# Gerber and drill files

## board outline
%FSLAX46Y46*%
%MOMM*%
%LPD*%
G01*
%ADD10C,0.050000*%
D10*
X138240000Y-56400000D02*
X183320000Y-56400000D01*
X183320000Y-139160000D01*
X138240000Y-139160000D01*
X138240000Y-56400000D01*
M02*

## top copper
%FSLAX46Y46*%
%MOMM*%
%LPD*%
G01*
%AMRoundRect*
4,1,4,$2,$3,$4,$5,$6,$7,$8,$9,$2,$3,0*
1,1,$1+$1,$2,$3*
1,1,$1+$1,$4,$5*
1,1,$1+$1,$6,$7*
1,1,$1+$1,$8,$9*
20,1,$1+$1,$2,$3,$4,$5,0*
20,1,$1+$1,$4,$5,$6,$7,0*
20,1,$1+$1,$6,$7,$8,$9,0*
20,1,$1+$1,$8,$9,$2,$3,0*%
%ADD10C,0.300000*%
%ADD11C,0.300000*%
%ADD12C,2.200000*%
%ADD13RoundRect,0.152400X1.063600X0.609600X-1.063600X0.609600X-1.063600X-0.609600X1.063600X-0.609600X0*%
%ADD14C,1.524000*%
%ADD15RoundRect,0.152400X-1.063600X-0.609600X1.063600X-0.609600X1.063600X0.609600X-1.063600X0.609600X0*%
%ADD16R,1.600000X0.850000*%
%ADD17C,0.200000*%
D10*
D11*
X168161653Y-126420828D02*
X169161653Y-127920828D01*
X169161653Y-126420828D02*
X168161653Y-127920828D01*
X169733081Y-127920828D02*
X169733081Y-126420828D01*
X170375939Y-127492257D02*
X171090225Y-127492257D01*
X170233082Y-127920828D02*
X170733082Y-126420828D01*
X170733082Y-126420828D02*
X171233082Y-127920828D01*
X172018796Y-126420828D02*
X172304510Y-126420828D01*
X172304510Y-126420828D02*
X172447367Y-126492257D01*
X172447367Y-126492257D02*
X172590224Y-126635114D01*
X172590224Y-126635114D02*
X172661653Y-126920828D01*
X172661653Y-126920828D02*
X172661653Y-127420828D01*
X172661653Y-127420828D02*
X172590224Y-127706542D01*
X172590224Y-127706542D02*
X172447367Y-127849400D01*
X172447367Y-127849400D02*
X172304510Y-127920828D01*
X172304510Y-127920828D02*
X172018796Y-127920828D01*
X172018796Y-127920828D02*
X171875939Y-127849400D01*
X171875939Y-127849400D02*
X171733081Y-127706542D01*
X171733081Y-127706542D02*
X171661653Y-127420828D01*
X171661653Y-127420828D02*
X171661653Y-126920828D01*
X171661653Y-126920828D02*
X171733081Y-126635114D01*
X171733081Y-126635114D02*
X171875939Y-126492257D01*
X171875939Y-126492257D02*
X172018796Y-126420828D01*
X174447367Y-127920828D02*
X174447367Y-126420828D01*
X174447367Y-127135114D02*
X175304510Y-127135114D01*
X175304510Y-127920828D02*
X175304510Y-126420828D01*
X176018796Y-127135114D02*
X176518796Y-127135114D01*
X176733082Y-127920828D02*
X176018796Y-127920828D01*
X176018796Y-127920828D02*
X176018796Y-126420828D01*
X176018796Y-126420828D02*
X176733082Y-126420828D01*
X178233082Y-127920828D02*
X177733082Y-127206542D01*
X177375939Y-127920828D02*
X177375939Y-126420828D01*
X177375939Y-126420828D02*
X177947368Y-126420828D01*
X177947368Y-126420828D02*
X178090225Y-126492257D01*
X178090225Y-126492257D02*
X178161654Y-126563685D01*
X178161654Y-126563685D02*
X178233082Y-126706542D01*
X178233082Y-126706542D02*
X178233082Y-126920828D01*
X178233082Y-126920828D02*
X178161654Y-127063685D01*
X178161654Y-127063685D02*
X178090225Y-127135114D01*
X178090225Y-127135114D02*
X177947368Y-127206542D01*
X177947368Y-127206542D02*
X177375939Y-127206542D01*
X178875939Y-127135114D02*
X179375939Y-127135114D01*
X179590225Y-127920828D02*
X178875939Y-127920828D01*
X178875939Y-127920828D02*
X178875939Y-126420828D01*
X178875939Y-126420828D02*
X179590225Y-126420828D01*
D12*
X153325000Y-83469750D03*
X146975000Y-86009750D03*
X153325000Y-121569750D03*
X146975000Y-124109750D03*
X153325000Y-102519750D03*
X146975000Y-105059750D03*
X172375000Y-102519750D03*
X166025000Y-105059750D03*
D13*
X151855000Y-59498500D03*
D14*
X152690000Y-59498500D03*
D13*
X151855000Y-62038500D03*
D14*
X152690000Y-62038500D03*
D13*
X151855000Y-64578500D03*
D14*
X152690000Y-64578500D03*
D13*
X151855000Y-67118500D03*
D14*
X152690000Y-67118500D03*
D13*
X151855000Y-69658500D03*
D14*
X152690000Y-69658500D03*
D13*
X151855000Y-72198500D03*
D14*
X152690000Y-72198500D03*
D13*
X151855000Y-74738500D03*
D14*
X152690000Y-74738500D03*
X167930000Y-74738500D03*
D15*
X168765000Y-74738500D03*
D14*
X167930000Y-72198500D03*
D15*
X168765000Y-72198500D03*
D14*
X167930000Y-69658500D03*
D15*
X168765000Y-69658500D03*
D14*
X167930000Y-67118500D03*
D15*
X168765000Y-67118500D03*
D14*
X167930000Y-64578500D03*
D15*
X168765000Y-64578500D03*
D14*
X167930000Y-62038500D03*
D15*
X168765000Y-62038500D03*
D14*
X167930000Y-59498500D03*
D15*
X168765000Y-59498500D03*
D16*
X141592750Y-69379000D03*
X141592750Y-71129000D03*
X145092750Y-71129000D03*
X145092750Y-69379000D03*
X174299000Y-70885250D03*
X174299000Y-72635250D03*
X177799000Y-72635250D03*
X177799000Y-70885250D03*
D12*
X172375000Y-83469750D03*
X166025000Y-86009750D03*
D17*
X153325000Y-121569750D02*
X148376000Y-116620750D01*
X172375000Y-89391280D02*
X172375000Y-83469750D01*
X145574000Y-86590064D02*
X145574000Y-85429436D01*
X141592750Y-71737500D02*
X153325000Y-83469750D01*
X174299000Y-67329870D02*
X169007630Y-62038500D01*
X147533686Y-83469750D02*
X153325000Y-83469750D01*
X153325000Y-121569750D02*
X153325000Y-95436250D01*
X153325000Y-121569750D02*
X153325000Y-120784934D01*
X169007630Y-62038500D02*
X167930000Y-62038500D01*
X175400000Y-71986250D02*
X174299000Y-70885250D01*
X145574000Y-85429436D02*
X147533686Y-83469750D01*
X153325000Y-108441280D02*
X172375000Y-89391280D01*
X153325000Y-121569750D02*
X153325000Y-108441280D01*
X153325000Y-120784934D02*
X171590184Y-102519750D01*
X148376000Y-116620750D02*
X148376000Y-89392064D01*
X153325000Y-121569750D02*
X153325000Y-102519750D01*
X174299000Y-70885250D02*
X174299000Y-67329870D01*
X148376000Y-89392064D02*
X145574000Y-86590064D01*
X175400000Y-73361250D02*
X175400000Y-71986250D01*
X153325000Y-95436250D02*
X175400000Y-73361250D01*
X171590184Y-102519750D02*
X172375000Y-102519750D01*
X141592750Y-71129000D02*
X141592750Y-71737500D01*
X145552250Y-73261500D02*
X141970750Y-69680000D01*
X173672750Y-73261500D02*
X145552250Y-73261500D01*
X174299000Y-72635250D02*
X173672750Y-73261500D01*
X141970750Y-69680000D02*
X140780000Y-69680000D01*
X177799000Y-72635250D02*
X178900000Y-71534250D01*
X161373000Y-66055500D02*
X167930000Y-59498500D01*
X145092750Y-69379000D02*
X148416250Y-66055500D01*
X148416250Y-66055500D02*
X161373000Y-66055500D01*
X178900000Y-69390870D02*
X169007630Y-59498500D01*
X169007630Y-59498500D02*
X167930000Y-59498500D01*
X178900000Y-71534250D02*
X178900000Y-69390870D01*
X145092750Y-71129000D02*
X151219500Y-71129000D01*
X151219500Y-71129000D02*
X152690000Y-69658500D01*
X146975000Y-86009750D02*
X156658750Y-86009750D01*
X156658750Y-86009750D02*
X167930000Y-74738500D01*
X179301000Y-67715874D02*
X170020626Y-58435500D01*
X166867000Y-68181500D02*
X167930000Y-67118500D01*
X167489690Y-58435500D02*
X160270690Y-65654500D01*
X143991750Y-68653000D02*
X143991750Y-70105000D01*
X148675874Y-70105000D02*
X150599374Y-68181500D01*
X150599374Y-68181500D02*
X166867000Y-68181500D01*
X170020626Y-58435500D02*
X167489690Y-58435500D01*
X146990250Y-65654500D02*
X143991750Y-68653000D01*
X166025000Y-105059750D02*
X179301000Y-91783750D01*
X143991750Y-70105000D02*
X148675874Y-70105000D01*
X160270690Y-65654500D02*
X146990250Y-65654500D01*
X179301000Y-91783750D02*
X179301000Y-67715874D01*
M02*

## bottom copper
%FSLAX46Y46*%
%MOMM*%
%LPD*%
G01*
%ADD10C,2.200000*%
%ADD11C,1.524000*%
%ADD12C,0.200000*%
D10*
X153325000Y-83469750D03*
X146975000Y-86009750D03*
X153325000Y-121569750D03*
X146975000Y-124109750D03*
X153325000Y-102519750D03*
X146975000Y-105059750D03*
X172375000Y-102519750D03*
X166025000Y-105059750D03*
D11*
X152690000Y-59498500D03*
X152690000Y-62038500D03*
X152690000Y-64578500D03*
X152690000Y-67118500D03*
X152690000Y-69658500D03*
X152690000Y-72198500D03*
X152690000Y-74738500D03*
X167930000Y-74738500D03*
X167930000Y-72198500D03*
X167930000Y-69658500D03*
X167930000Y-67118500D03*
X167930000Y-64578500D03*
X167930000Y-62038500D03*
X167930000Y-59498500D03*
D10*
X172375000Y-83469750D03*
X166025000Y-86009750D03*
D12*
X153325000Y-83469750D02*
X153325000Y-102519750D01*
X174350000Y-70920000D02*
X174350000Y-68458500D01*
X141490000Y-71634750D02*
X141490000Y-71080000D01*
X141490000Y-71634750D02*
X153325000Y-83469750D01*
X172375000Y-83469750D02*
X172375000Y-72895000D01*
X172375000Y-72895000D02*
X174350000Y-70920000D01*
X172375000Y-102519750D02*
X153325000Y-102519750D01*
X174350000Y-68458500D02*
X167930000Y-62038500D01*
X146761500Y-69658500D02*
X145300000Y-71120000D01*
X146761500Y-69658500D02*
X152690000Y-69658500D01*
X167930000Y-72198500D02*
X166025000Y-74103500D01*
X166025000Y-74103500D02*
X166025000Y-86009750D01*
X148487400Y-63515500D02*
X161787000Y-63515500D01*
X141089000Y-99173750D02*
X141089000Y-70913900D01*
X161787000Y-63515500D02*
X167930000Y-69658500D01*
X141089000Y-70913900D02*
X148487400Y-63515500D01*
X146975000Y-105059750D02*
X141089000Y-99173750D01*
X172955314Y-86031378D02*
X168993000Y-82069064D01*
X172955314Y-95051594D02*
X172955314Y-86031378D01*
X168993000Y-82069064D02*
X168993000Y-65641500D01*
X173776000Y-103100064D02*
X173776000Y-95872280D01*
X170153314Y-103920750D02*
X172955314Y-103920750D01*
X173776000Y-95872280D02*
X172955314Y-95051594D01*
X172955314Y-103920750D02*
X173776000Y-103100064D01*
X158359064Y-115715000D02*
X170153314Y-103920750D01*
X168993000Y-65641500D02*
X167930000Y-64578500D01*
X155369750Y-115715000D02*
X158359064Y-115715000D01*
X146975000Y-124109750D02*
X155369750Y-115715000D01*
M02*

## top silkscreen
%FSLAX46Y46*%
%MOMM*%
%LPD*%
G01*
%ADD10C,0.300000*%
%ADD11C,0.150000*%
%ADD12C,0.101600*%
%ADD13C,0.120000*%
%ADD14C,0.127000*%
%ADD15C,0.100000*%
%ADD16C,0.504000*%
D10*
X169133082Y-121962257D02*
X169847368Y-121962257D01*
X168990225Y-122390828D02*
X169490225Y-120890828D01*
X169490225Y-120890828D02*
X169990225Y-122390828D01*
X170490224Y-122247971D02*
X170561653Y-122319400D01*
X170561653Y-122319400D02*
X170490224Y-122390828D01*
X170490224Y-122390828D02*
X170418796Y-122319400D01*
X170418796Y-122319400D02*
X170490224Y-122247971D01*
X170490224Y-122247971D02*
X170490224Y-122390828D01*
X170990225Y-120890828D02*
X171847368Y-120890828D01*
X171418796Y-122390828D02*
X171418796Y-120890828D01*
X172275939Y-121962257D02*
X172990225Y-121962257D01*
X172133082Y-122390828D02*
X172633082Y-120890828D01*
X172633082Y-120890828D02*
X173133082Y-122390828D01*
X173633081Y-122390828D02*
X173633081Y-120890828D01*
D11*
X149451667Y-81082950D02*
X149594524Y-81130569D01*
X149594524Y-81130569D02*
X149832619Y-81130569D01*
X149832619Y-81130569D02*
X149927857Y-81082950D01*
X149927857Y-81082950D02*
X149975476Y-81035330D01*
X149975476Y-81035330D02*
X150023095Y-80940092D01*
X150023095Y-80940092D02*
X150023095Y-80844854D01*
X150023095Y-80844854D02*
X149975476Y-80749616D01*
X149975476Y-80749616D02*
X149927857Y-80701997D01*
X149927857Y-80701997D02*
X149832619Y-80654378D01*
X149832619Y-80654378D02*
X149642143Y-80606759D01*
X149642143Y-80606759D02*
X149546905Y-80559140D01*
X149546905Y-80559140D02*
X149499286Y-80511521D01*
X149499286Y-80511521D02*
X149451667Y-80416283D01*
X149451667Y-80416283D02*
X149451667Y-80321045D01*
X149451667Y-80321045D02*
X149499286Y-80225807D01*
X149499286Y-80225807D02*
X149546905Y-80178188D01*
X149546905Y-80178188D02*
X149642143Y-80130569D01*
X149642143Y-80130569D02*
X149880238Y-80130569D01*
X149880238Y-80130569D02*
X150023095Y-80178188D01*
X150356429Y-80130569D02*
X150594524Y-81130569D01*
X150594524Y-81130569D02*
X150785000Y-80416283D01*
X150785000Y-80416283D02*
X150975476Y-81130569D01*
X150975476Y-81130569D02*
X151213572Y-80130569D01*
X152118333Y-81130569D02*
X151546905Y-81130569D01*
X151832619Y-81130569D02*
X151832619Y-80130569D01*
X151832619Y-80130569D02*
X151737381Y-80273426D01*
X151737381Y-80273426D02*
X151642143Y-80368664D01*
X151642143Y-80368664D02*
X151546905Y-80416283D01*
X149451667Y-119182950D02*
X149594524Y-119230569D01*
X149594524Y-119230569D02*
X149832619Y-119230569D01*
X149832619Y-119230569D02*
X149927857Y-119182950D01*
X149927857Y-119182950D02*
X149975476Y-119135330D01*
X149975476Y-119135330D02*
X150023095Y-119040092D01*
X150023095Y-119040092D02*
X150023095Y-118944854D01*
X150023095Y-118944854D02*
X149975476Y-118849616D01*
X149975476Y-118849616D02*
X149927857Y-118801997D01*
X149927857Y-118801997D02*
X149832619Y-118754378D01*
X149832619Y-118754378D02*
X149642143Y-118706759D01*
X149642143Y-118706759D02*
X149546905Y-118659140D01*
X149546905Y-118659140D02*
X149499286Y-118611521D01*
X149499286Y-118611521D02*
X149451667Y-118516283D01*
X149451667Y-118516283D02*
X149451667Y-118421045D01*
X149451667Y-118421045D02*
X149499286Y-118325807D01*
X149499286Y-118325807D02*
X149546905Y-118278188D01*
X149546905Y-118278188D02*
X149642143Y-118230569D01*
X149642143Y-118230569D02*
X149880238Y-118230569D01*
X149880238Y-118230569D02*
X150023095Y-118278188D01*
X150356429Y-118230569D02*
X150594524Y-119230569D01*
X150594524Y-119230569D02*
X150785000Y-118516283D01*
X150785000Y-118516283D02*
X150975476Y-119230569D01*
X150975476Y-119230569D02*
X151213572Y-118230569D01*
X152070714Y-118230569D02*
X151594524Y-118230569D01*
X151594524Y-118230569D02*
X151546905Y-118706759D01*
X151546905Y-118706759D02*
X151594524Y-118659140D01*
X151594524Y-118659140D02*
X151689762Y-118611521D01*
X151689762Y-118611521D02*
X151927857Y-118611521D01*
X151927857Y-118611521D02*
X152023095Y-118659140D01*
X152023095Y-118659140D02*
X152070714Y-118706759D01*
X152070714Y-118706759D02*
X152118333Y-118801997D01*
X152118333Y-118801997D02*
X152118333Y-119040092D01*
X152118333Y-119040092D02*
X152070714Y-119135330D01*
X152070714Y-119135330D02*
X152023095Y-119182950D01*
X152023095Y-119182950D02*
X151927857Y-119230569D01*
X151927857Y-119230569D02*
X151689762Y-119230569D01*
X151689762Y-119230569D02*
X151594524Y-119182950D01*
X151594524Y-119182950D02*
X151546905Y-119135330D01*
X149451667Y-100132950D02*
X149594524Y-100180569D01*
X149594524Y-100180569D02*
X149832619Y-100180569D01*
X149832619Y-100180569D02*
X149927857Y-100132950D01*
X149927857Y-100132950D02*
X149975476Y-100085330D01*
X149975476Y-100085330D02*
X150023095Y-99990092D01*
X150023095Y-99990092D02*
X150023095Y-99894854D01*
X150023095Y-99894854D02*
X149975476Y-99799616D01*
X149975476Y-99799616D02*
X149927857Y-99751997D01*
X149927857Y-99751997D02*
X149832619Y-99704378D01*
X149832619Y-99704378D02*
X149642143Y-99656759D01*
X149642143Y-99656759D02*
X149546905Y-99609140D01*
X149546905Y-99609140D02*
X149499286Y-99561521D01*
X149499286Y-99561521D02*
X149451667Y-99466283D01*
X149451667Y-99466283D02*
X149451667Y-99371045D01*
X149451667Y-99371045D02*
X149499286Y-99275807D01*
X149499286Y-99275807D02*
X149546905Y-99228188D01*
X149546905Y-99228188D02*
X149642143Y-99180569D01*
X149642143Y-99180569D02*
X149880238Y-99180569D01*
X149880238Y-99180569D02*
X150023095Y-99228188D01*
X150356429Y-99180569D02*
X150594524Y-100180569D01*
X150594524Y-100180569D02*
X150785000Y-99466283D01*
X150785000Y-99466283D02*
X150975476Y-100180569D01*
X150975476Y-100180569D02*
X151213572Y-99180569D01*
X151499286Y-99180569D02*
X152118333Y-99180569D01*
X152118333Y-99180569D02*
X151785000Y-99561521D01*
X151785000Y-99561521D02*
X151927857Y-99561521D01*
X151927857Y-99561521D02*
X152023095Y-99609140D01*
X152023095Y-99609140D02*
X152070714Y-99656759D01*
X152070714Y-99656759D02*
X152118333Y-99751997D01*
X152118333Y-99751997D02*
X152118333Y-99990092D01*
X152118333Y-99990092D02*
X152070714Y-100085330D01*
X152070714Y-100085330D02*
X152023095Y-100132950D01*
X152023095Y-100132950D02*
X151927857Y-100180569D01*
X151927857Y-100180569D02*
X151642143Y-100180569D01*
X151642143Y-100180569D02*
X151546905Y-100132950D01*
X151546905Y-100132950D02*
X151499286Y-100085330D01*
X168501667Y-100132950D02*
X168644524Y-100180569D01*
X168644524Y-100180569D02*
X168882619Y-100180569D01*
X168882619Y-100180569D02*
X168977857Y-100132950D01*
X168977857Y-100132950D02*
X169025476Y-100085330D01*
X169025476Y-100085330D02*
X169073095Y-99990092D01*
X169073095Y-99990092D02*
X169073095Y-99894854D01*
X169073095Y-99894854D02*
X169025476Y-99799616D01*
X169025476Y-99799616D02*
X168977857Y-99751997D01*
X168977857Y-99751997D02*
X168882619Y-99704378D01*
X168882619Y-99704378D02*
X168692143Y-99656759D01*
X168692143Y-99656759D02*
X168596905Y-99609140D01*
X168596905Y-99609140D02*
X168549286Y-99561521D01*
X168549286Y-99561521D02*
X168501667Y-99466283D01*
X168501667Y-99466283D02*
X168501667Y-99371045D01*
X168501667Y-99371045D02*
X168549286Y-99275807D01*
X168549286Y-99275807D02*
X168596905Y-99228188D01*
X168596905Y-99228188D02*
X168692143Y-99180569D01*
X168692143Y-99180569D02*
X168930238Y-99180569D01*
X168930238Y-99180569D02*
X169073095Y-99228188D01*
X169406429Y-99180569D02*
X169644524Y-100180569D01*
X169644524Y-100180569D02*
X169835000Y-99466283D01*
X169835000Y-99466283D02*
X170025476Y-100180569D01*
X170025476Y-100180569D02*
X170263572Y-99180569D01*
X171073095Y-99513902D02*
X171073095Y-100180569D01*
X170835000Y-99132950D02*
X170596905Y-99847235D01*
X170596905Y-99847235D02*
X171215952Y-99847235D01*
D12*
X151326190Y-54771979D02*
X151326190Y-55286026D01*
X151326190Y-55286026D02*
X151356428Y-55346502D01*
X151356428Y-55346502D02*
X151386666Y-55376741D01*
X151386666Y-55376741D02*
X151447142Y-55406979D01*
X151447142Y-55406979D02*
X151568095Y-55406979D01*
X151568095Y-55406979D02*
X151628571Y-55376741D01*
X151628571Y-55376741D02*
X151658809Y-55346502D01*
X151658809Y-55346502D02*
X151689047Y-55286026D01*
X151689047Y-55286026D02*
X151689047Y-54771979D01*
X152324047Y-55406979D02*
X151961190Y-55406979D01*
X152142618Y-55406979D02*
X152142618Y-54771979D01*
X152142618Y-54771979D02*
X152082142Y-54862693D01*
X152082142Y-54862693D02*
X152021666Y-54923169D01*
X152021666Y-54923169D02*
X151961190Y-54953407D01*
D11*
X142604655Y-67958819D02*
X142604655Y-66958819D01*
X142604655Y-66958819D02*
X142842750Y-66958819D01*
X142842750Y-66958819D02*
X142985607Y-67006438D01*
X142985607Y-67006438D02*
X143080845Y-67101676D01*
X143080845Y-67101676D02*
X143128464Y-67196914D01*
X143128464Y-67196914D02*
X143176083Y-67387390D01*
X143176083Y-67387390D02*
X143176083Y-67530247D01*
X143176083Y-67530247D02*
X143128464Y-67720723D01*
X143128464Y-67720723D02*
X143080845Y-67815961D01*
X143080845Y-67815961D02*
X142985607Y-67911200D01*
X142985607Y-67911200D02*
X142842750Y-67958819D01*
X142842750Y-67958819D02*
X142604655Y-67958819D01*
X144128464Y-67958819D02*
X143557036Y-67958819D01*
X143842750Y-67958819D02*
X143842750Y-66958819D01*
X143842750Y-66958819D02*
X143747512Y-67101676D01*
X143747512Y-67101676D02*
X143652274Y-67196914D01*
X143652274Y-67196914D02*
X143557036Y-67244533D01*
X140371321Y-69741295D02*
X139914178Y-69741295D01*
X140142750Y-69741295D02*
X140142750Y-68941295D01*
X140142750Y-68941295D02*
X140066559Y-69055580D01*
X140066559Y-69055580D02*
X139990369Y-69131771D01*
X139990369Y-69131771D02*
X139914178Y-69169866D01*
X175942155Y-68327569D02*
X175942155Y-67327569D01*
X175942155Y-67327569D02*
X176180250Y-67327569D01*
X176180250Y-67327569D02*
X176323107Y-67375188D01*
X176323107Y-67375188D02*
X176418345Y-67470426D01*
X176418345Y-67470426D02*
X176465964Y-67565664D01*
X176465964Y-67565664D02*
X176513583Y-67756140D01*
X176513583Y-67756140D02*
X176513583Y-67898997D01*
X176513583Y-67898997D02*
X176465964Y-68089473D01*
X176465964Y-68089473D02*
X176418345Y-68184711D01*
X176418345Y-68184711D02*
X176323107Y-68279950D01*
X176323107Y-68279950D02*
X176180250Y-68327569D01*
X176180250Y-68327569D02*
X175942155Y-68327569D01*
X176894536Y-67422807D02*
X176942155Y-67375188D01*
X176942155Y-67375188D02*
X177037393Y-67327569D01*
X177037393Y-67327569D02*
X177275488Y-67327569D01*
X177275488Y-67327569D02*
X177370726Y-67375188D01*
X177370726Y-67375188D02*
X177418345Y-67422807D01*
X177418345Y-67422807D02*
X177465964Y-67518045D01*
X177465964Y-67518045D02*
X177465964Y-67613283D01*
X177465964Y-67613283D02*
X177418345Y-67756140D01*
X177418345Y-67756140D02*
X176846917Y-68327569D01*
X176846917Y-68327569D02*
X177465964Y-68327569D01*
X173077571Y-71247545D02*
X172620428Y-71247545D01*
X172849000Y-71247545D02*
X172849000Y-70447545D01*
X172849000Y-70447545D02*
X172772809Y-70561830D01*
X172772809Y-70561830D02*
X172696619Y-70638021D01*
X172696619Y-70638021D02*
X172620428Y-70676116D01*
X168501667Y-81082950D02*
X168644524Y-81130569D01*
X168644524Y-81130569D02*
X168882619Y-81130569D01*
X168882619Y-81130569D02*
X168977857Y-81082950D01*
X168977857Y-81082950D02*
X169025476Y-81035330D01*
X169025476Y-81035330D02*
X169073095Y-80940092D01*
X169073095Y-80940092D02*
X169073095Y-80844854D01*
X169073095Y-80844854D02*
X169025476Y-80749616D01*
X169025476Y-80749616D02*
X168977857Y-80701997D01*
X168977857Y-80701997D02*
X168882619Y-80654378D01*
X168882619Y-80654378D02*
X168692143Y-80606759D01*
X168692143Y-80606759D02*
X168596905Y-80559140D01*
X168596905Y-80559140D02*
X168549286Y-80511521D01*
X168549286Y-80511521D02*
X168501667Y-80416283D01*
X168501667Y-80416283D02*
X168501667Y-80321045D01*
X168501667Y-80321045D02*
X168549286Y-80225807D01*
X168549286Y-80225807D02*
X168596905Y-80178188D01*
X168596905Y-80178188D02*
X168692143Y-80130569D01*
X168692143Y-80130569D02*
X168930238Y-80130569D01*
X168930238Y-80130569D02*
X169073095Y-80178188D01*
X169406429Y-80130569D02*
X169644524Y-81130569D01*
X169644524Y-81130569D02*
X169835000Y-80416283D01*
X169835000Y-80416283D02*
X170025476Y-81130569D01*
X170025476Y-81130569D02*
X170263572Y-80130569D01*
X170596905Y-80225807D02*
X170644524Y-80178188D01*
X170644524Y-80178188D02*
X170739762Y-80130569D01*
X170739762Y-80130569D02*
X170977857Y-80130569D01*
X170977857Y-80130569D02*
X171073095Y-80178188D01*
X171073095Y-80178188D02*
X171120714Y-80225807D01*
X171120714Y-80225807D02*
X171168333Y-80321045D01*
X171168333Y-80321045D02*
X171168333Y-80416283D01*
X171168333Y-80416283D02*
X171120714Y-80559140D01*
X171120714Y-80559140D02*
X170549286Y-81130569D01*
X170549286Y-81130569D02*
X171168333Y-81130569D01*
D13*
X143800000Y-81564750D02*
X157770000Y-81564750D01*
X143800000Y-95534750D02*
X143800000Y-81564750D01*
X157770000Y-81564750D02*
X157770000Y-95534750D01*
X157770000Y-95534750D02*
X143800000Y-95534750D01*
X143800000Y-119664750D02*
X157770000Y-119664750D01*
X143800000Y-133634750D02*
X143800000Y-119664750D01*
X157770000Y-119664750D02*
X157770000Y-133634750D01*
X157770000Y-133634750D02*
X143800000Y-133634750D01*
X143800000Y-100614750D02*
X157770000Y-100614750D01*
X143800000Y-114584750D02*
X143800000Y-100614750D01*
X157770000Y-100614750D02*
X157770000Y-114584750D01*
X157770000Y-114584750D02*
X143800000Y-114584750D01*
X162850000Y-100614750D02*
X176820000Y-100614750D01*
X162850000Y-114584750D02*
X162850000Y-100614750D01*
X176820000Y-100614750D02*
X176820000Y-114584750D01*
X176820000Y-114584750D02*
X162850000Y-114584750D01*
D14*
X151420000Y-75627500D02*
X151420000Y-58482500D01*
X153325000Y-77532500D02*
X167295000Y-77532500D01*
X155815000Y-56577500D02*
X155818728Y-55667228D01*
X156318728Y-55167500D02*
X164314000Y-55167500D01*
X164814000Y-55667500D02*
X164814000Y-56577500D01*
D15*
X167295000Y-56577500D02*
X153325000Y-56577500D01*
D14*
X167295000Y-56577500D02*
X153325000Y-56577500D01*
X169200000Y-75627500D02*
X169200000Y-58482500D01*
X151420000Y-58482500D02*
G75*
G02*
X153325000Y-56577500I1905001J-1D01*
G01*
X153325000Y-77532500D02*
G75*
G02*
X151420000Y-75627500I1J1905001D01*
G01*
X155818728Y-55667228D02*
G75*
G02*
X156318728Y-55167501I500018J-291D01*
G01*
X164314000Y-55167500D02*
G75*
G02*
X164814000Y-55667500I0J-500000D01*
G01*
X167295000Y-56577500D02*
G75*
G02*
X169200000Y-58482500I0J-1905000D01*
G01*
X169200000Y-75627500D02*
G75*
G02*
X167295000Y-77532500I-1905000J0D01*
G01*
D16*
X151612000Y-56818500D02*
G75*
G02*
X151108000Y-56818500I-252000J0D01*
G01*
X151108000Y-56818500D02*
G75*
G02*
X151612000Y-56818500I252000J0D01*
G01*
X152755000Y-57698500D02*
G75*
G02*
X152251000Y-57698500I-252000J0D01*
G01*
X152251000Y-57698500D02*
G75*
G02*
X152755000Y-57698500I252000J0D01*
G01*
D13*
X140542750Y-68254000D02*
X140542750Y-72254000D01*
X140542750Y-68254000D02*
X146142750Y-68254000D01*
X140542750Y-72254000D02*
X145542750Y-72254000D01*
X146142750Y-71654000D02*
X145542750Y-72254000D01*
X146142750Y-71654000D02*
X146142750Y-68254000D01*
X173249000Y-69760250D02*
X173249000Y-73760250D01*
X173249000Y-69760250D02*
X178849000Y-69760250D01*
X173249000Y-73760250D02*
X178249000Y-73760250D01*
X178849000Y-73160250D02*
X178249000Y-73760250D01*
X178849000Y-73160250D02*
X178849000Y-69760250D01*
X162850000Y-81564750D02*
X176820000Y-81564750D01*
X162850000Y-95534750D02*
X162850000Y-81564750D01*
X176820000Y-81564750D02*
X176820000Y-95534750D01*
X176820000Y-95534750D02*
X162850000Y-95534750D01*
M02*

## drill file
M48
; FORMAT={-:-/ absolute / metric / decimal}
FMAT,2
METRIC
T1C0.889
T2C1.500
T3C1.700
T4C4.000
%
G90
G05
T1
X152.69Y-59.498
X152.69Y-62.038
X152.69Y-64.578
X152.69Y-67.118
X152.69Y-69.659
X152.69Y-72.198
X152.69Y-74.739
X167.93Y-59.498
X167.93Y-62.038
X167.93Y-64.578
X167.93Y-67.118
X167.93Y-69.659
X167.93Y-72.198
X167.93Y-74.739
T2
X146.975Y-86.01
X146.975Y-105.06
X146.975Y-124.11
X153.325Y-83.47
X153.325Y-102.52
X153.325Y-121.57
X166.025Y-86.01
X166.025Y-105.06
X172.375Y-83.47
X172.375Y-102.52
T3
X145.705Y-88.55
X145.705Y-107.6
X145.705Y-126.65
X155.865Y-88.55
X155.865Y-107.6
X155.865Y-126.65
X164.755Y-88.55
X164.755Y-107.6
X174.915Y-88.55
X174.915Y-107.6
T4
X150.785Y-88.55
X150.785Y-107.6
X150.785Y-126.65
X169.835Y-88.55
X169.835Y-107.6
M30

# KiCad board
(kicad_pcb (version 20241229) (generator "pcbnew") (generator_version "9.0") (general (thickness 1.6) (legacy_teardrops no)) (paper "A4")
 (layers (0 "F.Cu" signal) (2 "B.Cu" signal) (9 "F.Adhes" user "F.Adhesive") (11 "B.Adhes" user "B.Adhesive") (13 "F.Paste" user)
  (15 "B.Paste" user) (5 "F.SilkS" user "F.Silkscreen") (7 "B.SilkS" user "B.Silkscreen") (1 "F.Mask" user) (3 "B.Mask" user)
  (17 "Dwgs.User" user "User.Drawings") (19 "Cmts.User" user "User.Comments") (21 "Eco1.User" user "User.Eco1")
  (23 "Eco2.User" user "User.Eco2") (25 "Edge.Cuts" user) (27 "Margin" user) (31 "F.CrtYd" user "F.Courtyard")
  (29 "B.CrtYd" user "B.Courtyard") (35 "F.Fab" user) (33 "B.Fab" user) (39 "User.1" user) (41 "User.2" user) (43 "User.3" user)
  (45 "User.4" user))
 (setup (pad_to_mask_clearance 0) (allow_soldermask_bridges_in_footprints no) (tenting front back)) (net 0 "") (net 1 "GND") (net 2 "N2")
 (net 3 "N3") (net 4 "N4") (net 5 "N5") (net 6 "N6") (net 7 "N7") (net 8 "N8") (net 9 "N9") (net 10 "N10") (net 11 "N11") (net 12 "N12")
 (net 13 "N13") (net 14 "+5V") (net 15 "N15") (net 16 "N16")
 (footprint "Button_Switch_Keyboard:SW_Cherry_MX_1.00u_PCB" (layer "F.Cu") (at 153.325 83.46975)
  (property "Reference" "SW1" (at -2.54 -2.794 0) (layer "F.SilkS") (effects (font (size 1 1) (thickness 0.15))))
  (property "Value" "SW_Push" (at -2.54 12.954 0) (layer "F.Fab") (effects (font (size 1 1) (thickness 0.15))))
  (fp_line (start -9.525 -1.905) (end 4.445 -1.905) (stroke (width 0.12) (type solid)) (layer "F.SilkS"))
  (fp_line (start -9.525 12.065) (end -9.525 -1.905) (stroke (width 0.12) (type solid)) (layer "F.SilkS"))
  (fp_line (start 4.445 -1.905) (end 4.445 12.065) (stroke (width 0.12) (type solid)) (layer "F.SilkS"))
  (fp_line (start 4.445 12.065) (end -9.525 12.065) (stroke (width 0.12) (type solid)) (layer "F.SilkS"))
  (pad "" np_thru_hole circle (at -7.62 5.08) (size 1.7 1.7) (drill 1.7) (layers "*.Cu" "*.Mask"))
  (pad "" np_thru_hole circle (at -2.54 5.08) (size 4 4) (drill 4) (layers "*.Cu" "*.Mask"))
  (pad "" np_thru_hole circle (at 2.54 5.08) (size 1.7 1.7) (drill 1.7) (layers "*.Cu" "*.Mask"))
  (pad "1" thru_hole circle (at 0 0) (size 2.2 2.2) (drill 1.5) (layers "*.Cu" "*.Mask") (remove_unused_layers no) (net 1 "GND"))
  (pad "2" thru_hole circle (at -6.35 2.54) (size 2.2 2.2) (drill 1.5) (layers "*.Cu" "*.Mask") (remove_unused_layers no) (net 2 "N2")))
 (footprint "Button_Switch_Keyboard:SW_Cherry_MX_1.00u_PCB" (layer "F.Cu") (at 153.325 121.56975)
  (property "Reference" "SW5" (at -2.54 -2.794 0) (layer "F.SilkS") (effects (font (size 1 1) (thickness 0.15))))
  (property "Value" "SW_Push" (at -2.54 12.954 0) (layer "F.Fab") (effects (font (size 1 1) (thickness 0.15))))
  (fp_line (start -9.525 -1.905) (end 4.445 -1.905) (stroke (width 0.12) (type solid)) (layer "F.SilkS"))
  (fp_line (start -9.525 12.065) (end -9.525 -1.905) (stroke (width 0.12) (type solid)) (layer "F.SilkS"))
  (fp_line (start 4.445 -1.905) (end 4.445 12.065) (stroke (width 0.12) (type solid)) (layer "F.SilkS"))
  (fp_line (start 4.445 12.065) (end -9.525 12.065) (stroke (width 0.12) (type solid)) (layer "F.SilkS"))
  (pad "" np_thru_hole circle (at -7.62 5.08) (size 1.7 1.7) (drill 1.7) (layers "*.Cu" "*.Mask"))
  (pad "" np_thru_hole circle (at -2.54 5.08) (size 4 4) (drill 4) (layers "*.Cu" "*.Mask"))
  (pad "" np_thru_hole circle (at 2.54 5.08) (size 1.7 1.7) (drill 1.7) (layers "*.Cu" "*.Mask"))
  (pad "1" thru_hole circle (at 0 0) (size 2.2 2.2) (drill 1.5) (layers "*.Cu" "*.Mask") (remove_unused_layers no) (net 1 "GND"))
  (pad "2" thru_hole circle (at -6.35 2.54) (size 2.2 2.2) (drill 1.5) (layers "*.Cu" "*.Mask") (remove_unused_layers no) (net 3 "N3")))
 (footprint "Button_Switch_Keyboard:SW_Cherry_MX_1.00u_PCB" (layer "F.Cu") (at 153.325 102.51975)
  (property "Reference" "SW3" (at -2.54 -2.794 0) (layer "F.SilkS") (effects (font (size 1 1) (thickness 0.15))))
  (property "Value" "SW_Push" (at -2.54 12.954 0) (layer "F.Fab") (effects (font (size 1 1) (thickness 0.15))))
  (fp_line (start -9.525 -1.905) (end 4.445 -1.905) (stroke (width 0.12) (type solid)) (layer "F.SilkS"))
  (fp_line (start -9.525 12.065) (end -9.525 -1.905) (stroke (width 0.12) (type solid)) (layer "F.SilkS"))
  (fp_line (start 4.445 -1.905) (end 4.445 12.065) (stroke (width 0.12) (type solid)) (layer "F.SilkS"))
  (fp_line (start 4.445 12.065) (end -9.525 12.065) (stroke (width 0.12) (type solid)) (layer "F.SilkS"))
  (pad "" np_thru_hole circle (at -7.62 5.08) (size 1.7 1.7) (drill 1.7) (layers "*.Cu" "*.Mask"))
  (pad "" np_thru_hole circle (at -2.54 5.08) (size 4 4) (drill 4) (layers "*.Cu" "*.Mask"))
  (pad "" np_thru_hole circle (at 2.54 5.08) (size 1.7 1.7) (drill 1.7) (layers "*.Cu" "*.Mask"))
  (pad "1" thru_hole circle (at 0 0) (size 2.2 2.2) (drill 1.5) (layers "*.Cu" "*.Mask") (remove_unused_layers no) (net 1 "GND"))
  (pad "2" thru_hole circle (at -6.35 2.54) (size 2.2 2.2) (drill 1.5) (layers "*.Cu" "*.Mask") (remove_unused_layers no) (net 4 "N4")))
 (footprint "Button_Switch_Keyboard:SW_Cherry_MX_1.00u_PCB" (layer "F.Cu") (at 172.375 102.51975)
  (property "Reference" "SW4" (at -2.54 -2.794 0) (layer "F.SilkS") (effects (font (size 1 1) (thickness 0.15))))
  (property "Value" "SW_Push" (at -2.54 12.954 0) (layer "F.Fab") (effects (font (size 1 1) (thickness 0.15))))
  (fp_line (start -9.525 -1.905) (end 4.445 -1.905) (stroke (width 0.12) (type solid)) (layer "F.SilkS"))
  (fp_line (start -9.525 12.065) (end -9.525 -1.905) (stroke (width 0.12) (type solid)) (layer "F.SilkS"))
  (fp_line (start 4.445 -1.905) (end 4.445 12.065) (stroke (width 0.12) (type solid)) (layer "F.SilkS"))
  (fp_line (start 4.445 12.065) (end -9.525 12.065) (stroke (width 0.12) (type solid)) (layer "F.SilkS"))
  (pad "" np_thru_hole circle (at -7.62 5.08) (size 1.7 1.7) (drill 1.7) (layers "*.Cu" "*.Mask"))
  (pad "" np_thru_hole circle (at -2.54 5.08) (size 4 4) (drill 4) (layers "*.Cu" "*.Mask"))
  (pad "" np_thru_hole circle (at 2.54 5.08) (size 1.7 1.7) (drill 1.7) (layers "*.Cu" "*.Mask"))
  (pad "1" thru_hole circle (at 0 0) (size 2.2 2.2) (drill 1.5) (layers "*.Cu" "*.Mask") (remove_unused_layers no) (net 1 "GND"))
  (pad "2" thru_hole circle (at -6.35 2.54) (size 2.2 2.2) (drill 1.5) (layers "*.Cu" "*.Mask") (remove_unused_layers no) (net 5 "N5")))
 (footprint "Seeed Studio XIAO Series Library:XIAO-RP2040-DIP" (layer "F.Cu") (at 160.31 67.1185)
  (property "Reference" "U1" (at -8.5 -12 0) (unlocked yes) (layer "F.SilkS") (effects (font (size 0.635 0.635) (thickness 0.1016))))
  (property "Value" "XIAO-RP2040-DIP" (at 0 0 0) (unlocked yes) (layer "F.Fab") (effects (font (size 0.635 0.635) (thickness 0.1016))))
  (fp_line (start -8.89 8.509) (end -8.89 -8.636) (stroke (width 0.127) (type solid)) (layer "F.SilkS"))
  (fp_line (start -6.985 10.414) (end 6.985 10.414) (stroke (width 0.127) (type solid)) (layer "F.SilkS"))
  (fp_line (start -4.495 -10.541) (end -4.491272 -11.451272) (stroke (width 0.127) (type solid)) (layer "F.SilkS"))
  (fp_line (start -3.991272 -11.951) (end 4.004 -11.951) (stroke (width 0.127) (type solid)) (layer "F.SilkS"))
  (fp_line (start 4.504 -11.451) (end 4.504 -10.541) (stroke (width 0.127) (type solid)) (layer "F.SilkS"))
  (fp_line (start 6.985 -10.541) (end -6.985 -10.541) (stroke (width 0.1) (type solid)) (layer "F.SilkS"))
  (fp_line (start 6.985 -10.541) (end -6.985 -10.541) (stroke (width 0.127) (type solid)) (layer "F.SilkS"))
  (fp_line (start 8.89 8.509) (end 8.89 -8.636) (stroke (width 0.127) (type solid)) (layer "F.SilkS"))
  (fp_arc (start -8.89 -8.636) (mid -8.332038 -9.983038) (end -6.985 -10.541) (stroke (width 0.127) (type solid)) (layer "F.SilkS"))
  (fp_arc (start -6.985 10.414) (mid -8.332038 9.856038) (end -8.89 8.509) (stroke (width 0.127) (type solid)) (layer "F.SilkS"))
  (fp_arc (start -4.491272 -11.451272) (mid -4.344728 -11.80464) (end -3.991272 -11.951) (stroke (width 0.127) (type default))
   (layer "F.SilkS"))
  (fp_arc (start 4.004 -11.951) (mid 4.357553 -11.804553) (end 4.504 -11.451) (stroke (width 0.127) (type default)) (layer "F.SilkS"))
  (fp_arc (start 6.985 -10.541) (mid 8.332038 -9.983038) (end 8.89 -8.636) (stroke (width 0.127) (type solid)) (layer "F.SilkS"))
  (fp_arc (start 8.89 8.509) (mid 8.332038 9.856038) (end 6.985 10.414) (stroke (width 0.127) (type solid)) (layer "F.SilkS"))
  (fp_circle (center -8.95 -10.3) (end -8.95 -10.554) (stroke (width 0.5) (type solid)) (fill yes) (layer "F.SilkS"))
  (fp_circle (center -7.807 -9.42) (end -7.807 -9.674) (stroke (width 0.5) (type solid)) (fill yes) (layer "F.SilkS"))
  (pad "1" smd roundrect (at -8.455 -7.62 180) (size 2.432 1.524) (layers "F.Cu" "F.Mask") (roundrect_rratio 0.1) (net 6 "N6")
   (thermal_bridge_angle 45))
  (pad "1" thru_hole circle (at -7.62 -7.62 180) (size 1.524 1.524) (drill 0.889) (layers "*.Cu" "*.Mask") (remove_unused_layers no)
   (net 6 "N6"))
  (pad "2" smd roundrect (at -8.455 -5.08 180) (size 2.432 1.524) (layers "F.Cu" "F.Mask") (roundrect_rratio 0.1) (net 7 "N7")
   (thermal_bridge_angle 45))
  (pad "2" thru_hole circle (at -7.62 -5.08 180) (size 1.524 1.524) (drill 0.889) (layers "*.Cu" "*.Mask") (remove_unused_layers no)
   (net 7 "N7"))
  (pad "3" smd roundrect (at -8.455 -2.54 180) (size 2.432 1.524) (layers "F.Cu" "F.Mask") (roundrect_rratio 0.1) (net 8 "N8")
   (thermal_bridge_angle 45))
  (pad "3" thru_hole circle (at -7.62 -2.54 180) (size 1.524 1.524) (drill 0.889) (layers "*.Cu" "*.Mask") (remove_unused_layers no)
   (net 8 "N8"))
  (pad "4" smd roundrect (at -8.455 0 180) (size 2.432 1.524) (layers "F.Cu" "F.Mask") (roundrect_rratio 0.1) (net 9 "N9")
   (thermal_bridge_angle 45))
  (pad "4" thru_hole circle (at -7.62 0 180) (size 1.524 1.524) (drill 0.889) (layers "*.Cu" "*.Mask") (remove_unused_layers no)
   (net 9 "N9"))
  (pad "5" smd roundrect (at -8.455 2.54 180) (size 2.432 1.524) (layers "F.Cu" "F.Mask") (roundrect_rratio 0.1) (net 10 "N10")
   (thermal_bridge_angle 45))
  (pad "5" thru_hole circle (at -7.62 2.54 180) (size 1.524 1.524) (drill 0.889) (layers "*.Cu" "*.Mask") (remove_unused_layers no)
   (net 10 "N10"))
  (pad "6" smd roundrect (at -8.455 5.08 180) (size 2.432 1.524) (layers "F.Cu" "F.Mask") (roundrect_rratio 0.1) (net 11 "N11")
   (thermal_bridge_angle 45))
  (pad "6" thru_hole circle (at -7.62 5.08 180) (size 1.524 1.524) (drill 0.889) (layers "*.Cu" "*.Mask") (remove_unused_layers no)
   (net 11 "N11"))
  (pad "7" smd roundrect (at -8.455 7.62 180) (size 2.432 1.524) (layers "F.Cu" "F.Mask") (roundrect_rratio 0.1) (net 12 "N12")
   (thermal_bridge_angle 45))
  (pad "7" thru_hole circle (at -7.62 7.62 180) (size 1.524 1.524) (drill 0.889) (layers "*.Cu" "*.Mask") (remove_unused_layers no)
   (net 12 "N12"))
  (pad "8" thru_hole circle (at 7.62 7.62) (size 1.524 1.524) (drill 0.889) (layers "*.Cu" "*.Mask") (remove_unused_layers no) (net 2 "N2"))
  (pad "8" smd roundrect (at 8.455 7.62) (size 2.432 1.524) (layers "F.Cu" "F.Mask") (roundrect_rratio 0.1) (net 2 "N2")
   (thermal_bridge_angle 45))
  (pad "9" thru_hole circle (at 7.62 5.08) (size 1.524 1.524) (drill 0.889) (layers "*.Cu" "*.Mask") (remove_unused_layers no)
   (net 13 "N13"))
  (pad "9" smd roundrect (at 8.455 5.08) (size 2.432 1.524) (layers "F.Cu" "F.Mask") (roundrect_rratio 0.1) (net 13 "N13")
   (thermal_bridge_angle 45))
  (pad "10" thru_hole circle (at 7.62 2.54) (size 1.524 1.524) (drill 0.889) (layers "*.Cu" "*.Mask") (remove_unused_layers no) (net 4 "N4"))
  (pad "10" smd roundrect (at 8.455 2.54) (size 2.432 1.524) (layers "F.Cu" "F.Mask") (roundrect_rratio 0.1) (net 4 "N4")
   (thermal_bridge_angle 45))
  (pad "11" thru_hole circle (at 7.62 0) (size 1.524 1.524) (drill 0.889) (layers "*.Cu" "*.Mask") (remove_unused_layers no) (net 5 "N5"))
  (pad "11" smd roundrect (at 8.455 0) (size 2.432 1.524) (layers "F.Cu" "F.Mask") (roundrect_rratio 0.1) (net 5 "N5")
   (thermal_bridge_angle 45))
  (pad "12" thru_hole circle (at 7.62 -2.54) (size 1.524 1.524) (drill 0.889) (layers "*.Cu" "*.Mask") (remove_unused_layers no)
   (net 3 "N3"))
  (pad "12" smd roundrect (at 8.455 -2.54) (size 2.432 1.524) (layers "F.Cu" "F.Mask") (roundrect_rratio 0.1) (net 3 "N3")
   (thermal_bridge_angle 45))
  (pad "13" thru_hole circle (at 7.62 -5.08) (size 1.524 1.524) (drill 0.889) (layers "*.Cu" "*.Mask") (remove_unused_layers no)
   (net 1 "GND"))
  (pad "13" smd roundrect (at 8.455 -5.08) (size 2.432 1.524) (layers "F.Cu" "F.Mask") (roundrect_rratio 0.1) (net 1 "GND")
   (thermal_bridge_angle 45))
  (pad "14" thru_hole circle (at 7.62 -7.62) (size 1.524 1.524) (drill 0.889) (layers "*.Cu" "*.Mask") (remove_unused_layers no)
   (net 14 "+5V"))
  (pad "14" smd roundrect (at 8.455 -7.62) (size 2.432 1.524) (layers "F.Cu" "F.Mask") (roundrect_rratio 0.1) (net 14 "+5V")
   (thermal_bridge_angle 45)))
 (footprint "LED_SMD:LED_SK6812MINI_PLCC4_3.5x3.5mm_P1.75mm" (layer "F.Cu") (at 143.34275 70.254)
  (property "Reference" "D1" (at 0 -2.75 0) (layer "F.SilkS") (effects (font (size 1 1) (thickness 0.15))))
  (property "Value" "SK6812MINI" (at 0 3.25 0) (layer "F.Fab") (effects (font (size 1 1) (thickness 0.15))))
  (fp_line (start -2.8 -2) (end -2.8 2) (stroke (width 0.12) (type default)) (layer "F.SilkS"))
  (fp_line (start -2.8 -2) (end 2.8 -2) (stroke (width 0.12) (type solid)) (layer "F.SilkS"))
  (fp_line (start -2.8 2) (end 2.2 2) (stroke (width 0.12) (type solid)) (layer "F.SilkS"))
  (fp_line (start 2.8 1.4) (end 2.2 2) (stroke (width 0.12) (type default)) (layer "F.SilkS"))
  (fp_line (start 2.8 1.4) (end 2.8 -2) (stroke (width 0.12) (type solid)) (layer "F.SilkS"))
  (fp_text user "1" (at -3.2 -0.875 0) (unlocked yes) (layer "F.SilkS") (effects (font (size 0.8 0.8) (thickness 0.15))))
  (pad "1" smd rect (at -1.75 -0.875) (size 1.6 0.85) (layers "F.Cu" "F.Mask" "F.Paste") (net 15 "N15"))
  (pad "2" smd rect (at -1.75 0.875) (size 1.6 0.85) (layers "F.Cu" "F.Mask" "F.Paste") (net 1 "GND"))
  (pad "3" smd rect (at 1.75 0.875) (size 1.6 0.85) (layers "F.Cu" "F.Mask" "F.Paste") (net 10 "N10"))
  (pad "4" smd rect (at 1.75 -0.875) (size 1.6 0.85) (layers "F.Cu" "F.Mask" "F.Paste") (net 14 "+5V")))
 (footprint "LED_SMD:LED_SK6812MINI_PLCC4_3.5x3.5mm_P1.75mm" (layer "F.Cu") (at 176.049 71.76025)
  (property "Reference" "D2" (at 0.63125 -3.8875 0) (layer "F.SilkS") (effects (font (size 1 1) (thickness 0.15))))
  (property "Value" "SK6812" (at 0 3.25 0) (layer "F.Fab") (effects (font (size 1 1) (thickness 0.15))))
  (fp_line (start -2.8 -2) (end -2.8 2) (stroke (width 0.12) (type default)) (layer "F.SilkS"))
  (fp_line (start -2.8 -2) (end 2.8 -2) (stroke (width 0.12) (type solid)) (layer "F.SilkS"))
  (fp_line (start -2.8 2) (end 2.2 2) (stroke (width 0.12) (type solid)) (layer "F.SilkS"))
  (fp_line (start 2.8 1.4) (end 2.2 2) (stroke (width 0.12) (type default)) (layer "F.SilkS"))
  (fp_line (start 2.8 1.4) (end 2.8 -2) (stroke (width 0.12) (type solid)) (layer "F.SilkS"))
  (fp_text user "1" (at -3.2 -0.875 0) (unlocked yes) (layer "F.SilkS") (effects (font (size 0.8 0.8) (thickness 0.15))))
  (pad "1" smd rect (at -1.75 -0.875) (size 1.6 0.85) (layers "F.Cu" "F.Mask" "F.Paste") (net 1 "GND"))
  (pad "2" smd rect (at -1.75 0.875) (size 1.6 0.85) (layers "F.Cu" "F.Mask" "F.Paste") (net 15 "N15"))
  (pad "3" smd rect (at 1.75 0.875) (size 1.6 0.85) (layers "F.Cu" "F.Mask" "F.Paste") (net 14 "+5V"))
  (pad "4" smd rect (at 1.75 -0.875) (size 1.6 0.85) (layers "F.Cu" "F.Mask" "F.Paste") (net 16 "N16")))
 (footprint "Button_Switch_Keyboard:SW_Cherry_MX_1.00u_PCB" (layer "F.Cu") (at 172.375 83.46975)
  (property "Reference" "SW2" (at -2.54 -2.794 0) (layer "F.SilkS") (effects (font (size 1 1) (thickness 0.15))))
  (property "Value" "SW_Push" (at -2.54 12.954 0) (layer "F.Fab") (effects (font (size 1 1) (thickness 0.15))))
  (fp_line (start -9.525 -1.905) (end 4.445 -1.905) (stroke (width 0.12) (type solid)) (layer "F.SilkS"))
  (fp_line (start -9.525 12.065) (end -9.525 -1.905) (stroke (width 0.12) (type solid)) (layer "F.SilkS"))
  (fp_line (start 4.445 -1.905) (end 4.445 12.065) (stroke (width 0.12) (type solid)) (layer "F.SilkS"))
  (fp_line (start 4.445 12.065) (end -9.525 12.065) (stroke (width 0.12) (type solid)) (layer "F.SilkS"))
  (pad "" np_thru_hole circle (at -7.62 5.08) (size 1.7 1.7) (drill 1.7) (layers "*.Cu" "*.Mask"))
  (pad "" np_thru_hole circle (at -2.54 5.08) (size 4 4) (drill 4) (layers "*.Cu" "*.Mask"))
  (pad "" np_thru_hole circle (at 2.54 5.08) (size 1.7 1.7) (drill 1.7) (layers "*.Cu" "*.Mask"))
  (pad "1" thru_hole circle (at 0 0) (size 2.2 2.2) (drill 1.5) (layers "*.Cu" "*.Mask") (remove_unused_layers no) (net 1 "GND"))
  (pad "2" thru_hole circle (at -6.35 2.54) (size 2.2 2.2) (drill 1.5) (layers "*.Cu" "*.Mask") (remove_unused_layers no) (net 13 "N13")))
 (gr_rect (start 138.24 56.4) (end 183.32 139.16) (stroke (width 0.05) (type solid)) (fill no) (layer "Edge.Cuts"))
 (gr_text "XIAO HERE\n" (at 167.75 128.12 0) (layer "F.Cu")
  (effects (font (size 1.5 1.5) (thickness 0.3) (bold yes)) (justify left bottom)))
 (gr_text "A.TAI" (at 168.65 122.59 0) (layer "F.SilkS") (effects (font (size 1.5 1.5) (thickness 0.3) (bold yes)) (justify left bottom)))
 (segment (start 153.325 121.56975) (end 148.376 116.62075) (width 0.2) (layer "F.Cu") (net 1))
 (segment (start 172.375 89.39128) (end 172.375 83.46975) (width 0.2) (layer "F.Cu") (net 1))
 (segment (start 145.574 86.590064) (end 145.574 85.429436) (width 0.2) (layer "F.Cu") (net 1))
 (segment (start 141.59275 71.7375) (end 153.325 83.46975) (width 0.2) (layer "F.Cu") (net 1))
 (segment (start 174.299 67.32987) (end 169.00763 62.0385) (width 0.2) (layer "F.Cu") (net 1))
 (segment (start 147.533686 83.46975) (end 153.325 83.46975) (width 0.2) (layer "F.Cu") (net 1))
 (segment (start 153.325 121.56975) (end 153.325 95.43625) (width 0.2) (layer "F.Cu") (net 1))
 (segment (start 153.325 121.56975) (end 153.325 120.784934) (width 0.2) (layer "F.Cu") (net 1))
 (segment (start 169.00763 62.0385) (end 167.93 62.0385) (width 0.2) (layer "F.Cu") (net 1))
 (segment (start 175.4 71.98625) (end 174.299 70.88525) (width 0.2) (layer "F.Cu") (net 1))
 (segment (start 145.574 85.429436) (end 147.533686 83.46975) (width 0.2) (layer "F.Cu") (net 1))
 (segment (start 153.325 108.44128) (end 172.375 89.39128) (width 0.2) (layer "F.Cu") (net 1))
 (segment (start 153.325 121.56975) (end 153.325 108.44128) (width 0.2) (layer "F.Cu") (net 1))
 (segment (start 153.325 120.784934) (end 171.590184 102.51975) (width 0.2) (layer "F.Cu") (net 1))
 (segment (start 148.376 116.62075) (end 148.376 89.392064) (width 0.2) (layer "F.Cu") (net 1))
 (segment (start 153.325 121.56975) (end 153.325 102.51975) (width 0.2) (layer "F.Cu") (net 1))
 (segment (start 174.299 70.88525) (end 174.299 67.32987) (width 0.2) (layer "F.Cu") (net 1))
 (segment (start 148.376 89.392064) (end 145.574 86.590064) (width 0.2) (layer "F.Cu") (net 1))
 (segment (start 175.4 73.36125) (end 175.4 71.98625) (width 0.2) (layer "F.Cu") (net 1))
 (segment (start 153.325 95.43625) (end 175.4 73.36125) (width 0.2) (layer "F.Cu") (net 1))
 (segment (start 171.590184 102.51975) (end 172.375 102.51975) (width 0.2) (layer "F.Cu") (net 1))
 (segment (start 141.59275 71.129) (end 141.59275 71.7375) (width 0.2) (layer "F.Cu") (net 1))
 (segment (start 153.325 83.46975) (end 153.325 102.51975) (width 0.2) (layer "B.Cu") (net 1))
 (segment (start 174.35 70.92) (end 174.35 68.4585) (width 0.2) (layer "B.Cu") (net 1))
 (segment (start 141.49 71.63475) (end 141.49 71.08) (width 0.2) (layer "B.Cu") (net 1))
 (segment (start 141.49 71.63475) (end 153.325 83.46975) (width 0.2) (layer "B.Cu") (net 1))
 (segment (start 172.375 83.46975) (end 172.375 72.895) (width 0.2) (layer "B.Cu") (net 1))
 (segment (start 172.375 72.895) (end 174.35 70.92) (width 0.2) (layer "B.Cu") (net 1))
 (segment (start 172.375 102.51975) (end 153.325 102.51975) (width 0.2) (layer "B.Cu") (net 1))
 (segment (start 174.35 68.4585) (end 167.93 62.0385) (width 0.2) (layer "B.Cu") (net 1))
 (segment (start 145.55225 73.2615) (end 141.97075 69.68) (width 0.2) (layer "F.Cu") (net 15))
 (segment (start 173.67275 73.2615) (end 145.55225 73.2615) (width 0.2) (layer "F.Cu") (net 15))
 (segment (start 174.299 72.63525) (end 173.67275 73.2615) (width 0.2) (layer "F.Cu") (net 15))
 (segment (start 141.97075 69.68) (end 140.78 69.68) (width 0.2) (layer "F.Cu") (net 15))
 (segment (start 177.799 72.63525) (end 178.9 71.53425) (width 0.2) (layer "F.Cu") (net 14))
 (segment (start 161.373 66.0555) (end 167.93 59.4985) (width 0.2) (layer "F.Cu") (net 14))
 (segment (start 145.09275 69.379) (end 148.41625 66.0555) (width 0.2) (layer "F.Cu") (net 14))
 (segment (start 148.41625 66.0555) (end 161.373 66.0555) (width 0.2) (layer "F.Cu") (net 14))
 (segment (start 178.9 69.39087) (end 169.00763 59.4985) (width 0.2) (layer "F.Cu") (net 14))
 (segment (start 169.00763 59.4985) (end 167.93 59.4985) (width 0.2) (layer "F.Cu") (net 14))
 (segment (start 178.9 71.53425) (end 178.9 69.39087) (width 0.2) (layer "F.Cu") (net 14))
 (segment (start 145.09275 71.129) (end 151.2195 71.129) (width 0.2) (layer "F.Cu") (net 10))
 (segment (start 151.2195 71.129) (end 152.69 69.6585) (width 0.2) (layer "F.Cu") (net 10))
 (segment (start 146.7615 69.6585) (end 145.3 71.12) (width 0.2) (layer "B.Cu") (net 10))
 (segment (start 146.7615 69.6585) (end 152.69 69.6585) (width 0.2) (layer "B.Cu") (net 10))
 (segment (start 146.975 86.00975) (end 156.65875 86.00975) (width 0.2) (layer "F.Cu") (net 2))
 (segment (start 156.65875 86.00975) (end 167.93 74.7385) (width 0.2) (layer "F.Cu") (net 2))
 (segment (start 167.93 72.1985) (end 166.025 74.1035) (width 0.2) (layer "B.Cu") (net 13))
 (segment (start 166.025 74.1035) (end 166.025 86.00975) (width 0.2) (layer "B.Cu") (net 13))
 (segment (start 148.4874 63.5155) (end 161.787 63.5155) (width 0.2) (layer "B.Cu") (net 4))
 (segment (start 141.089 99.17375) (end 141.089 70.9139) (width 0.2) (layer "B.Cu") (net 4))
 (segment (start 161.787 63.5155) (end 167.93 69.6585) (width 0.2) (layer "B.Cu") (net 4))
 (segment (start 141.089 70.9139) (end 148.4874 63.5155) (width 0.2) (layer "B.Cu") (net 4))
 (segment (start 146.975 105.05975) (end 141.089 99.17375) (width 0.2) (layer "B.Cu") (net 4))
 (segment (start 179.301 67.715874) (end 170.020626 58.4355) (width 0.2) (layer "F.Cu") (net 5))
 (segment (start 166.867 68.1815) (end 167.93 67.1185) (width 0.2) (layer "F.Cu") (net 5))
 (segment (start 167.48969 58.4355) (end 160.27069 65.6545) (width 0.2) (layer "F.Cu") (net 5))
 (segment (start 143.99175 68.653) (end 143.99175 70.105) (width 0.2) (layer "F.Cu") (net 5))
 (segment (start 148.675874 70.105) (end 150.599374 68.1815) (width 0.2) (layer "F.Cu") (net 5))
 (segment (start 150.599374 68.1815) (end 166.867 68.1815) (width 0.2) (layer "F.Cu") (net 5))
 (segment (start 170.020626 58.4355) (end 167.48969 58.4355) (width 0.2) (layer "F.Cu") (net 5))
 (segment (start 146.99025 65.6545) (end 143.99175 68.653) (width 0.2) (layer "F.Cu") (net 5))
 (segment (start 166.025 105.05975) (end 179.301 91.78375) (width 0.2) (layer "F.Cu") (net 5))
 (segment (start 143.99175 70.105) (end 148.675874 70.105) (width 0.2) (layer "F.Cu") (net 5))
 (segment (start 160.27069 65.6545) (end 146.99025 65.6545) (width 0.2) (layer "F.Cu") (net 5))
 (segment (start 179.301 91.78375) (end 179.301 67.715874) (width 0.2) (layer "F.Cu") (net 5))
 (segment (start 172.955314 86.031378) (end 168.993 82.069064) (width 0.2) (layer "B.Cu") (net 3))
 (segment (start 172.955314 95.051594) (end 172.955314 86.031378) (width 0.2) (layer "B.Cu") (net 3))
 (segment (start 168.993 82.069064) (end 168.993 65.6415) (width 0.2) (layer "B.Cu") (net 3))
 (segment (start 173.776 103.100064) (end 173.776 95.87228) (width 0.2) (layer "B.Cu") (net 3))
 (segment (start 170.153314 103.92075) (end 172.955314 103.92075) (width 0.2) (layer "B.Cu") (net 3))
 (segment (start 173.776 95.87228) (end 172.955314 95.051594) (width 0.2) (layer "B.Cu") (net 3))
 (segment (start 172.955314 103.92075) (end 173.776 103.100064) (width 0.2) (layer "B.Cu") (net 3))
 (segment (start 158.359064 115.715) (end 170.153314 103.92075) (width 0.2) (layer "B.Cu") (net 3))
 (segment (start 168.993 65.6415) (end 167.93 64.5785) (width 0.2) (layer "B.Cu") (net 3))
 (segment (start 155.36975 115.715) (end 158.359064 115.715) (width 0.2) (layer "B.Cu") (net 3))
 (segment (start 146.975 124.10975) (end 155.36975 115.715) (width 0.2) (layer "B.Cu") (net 3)))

